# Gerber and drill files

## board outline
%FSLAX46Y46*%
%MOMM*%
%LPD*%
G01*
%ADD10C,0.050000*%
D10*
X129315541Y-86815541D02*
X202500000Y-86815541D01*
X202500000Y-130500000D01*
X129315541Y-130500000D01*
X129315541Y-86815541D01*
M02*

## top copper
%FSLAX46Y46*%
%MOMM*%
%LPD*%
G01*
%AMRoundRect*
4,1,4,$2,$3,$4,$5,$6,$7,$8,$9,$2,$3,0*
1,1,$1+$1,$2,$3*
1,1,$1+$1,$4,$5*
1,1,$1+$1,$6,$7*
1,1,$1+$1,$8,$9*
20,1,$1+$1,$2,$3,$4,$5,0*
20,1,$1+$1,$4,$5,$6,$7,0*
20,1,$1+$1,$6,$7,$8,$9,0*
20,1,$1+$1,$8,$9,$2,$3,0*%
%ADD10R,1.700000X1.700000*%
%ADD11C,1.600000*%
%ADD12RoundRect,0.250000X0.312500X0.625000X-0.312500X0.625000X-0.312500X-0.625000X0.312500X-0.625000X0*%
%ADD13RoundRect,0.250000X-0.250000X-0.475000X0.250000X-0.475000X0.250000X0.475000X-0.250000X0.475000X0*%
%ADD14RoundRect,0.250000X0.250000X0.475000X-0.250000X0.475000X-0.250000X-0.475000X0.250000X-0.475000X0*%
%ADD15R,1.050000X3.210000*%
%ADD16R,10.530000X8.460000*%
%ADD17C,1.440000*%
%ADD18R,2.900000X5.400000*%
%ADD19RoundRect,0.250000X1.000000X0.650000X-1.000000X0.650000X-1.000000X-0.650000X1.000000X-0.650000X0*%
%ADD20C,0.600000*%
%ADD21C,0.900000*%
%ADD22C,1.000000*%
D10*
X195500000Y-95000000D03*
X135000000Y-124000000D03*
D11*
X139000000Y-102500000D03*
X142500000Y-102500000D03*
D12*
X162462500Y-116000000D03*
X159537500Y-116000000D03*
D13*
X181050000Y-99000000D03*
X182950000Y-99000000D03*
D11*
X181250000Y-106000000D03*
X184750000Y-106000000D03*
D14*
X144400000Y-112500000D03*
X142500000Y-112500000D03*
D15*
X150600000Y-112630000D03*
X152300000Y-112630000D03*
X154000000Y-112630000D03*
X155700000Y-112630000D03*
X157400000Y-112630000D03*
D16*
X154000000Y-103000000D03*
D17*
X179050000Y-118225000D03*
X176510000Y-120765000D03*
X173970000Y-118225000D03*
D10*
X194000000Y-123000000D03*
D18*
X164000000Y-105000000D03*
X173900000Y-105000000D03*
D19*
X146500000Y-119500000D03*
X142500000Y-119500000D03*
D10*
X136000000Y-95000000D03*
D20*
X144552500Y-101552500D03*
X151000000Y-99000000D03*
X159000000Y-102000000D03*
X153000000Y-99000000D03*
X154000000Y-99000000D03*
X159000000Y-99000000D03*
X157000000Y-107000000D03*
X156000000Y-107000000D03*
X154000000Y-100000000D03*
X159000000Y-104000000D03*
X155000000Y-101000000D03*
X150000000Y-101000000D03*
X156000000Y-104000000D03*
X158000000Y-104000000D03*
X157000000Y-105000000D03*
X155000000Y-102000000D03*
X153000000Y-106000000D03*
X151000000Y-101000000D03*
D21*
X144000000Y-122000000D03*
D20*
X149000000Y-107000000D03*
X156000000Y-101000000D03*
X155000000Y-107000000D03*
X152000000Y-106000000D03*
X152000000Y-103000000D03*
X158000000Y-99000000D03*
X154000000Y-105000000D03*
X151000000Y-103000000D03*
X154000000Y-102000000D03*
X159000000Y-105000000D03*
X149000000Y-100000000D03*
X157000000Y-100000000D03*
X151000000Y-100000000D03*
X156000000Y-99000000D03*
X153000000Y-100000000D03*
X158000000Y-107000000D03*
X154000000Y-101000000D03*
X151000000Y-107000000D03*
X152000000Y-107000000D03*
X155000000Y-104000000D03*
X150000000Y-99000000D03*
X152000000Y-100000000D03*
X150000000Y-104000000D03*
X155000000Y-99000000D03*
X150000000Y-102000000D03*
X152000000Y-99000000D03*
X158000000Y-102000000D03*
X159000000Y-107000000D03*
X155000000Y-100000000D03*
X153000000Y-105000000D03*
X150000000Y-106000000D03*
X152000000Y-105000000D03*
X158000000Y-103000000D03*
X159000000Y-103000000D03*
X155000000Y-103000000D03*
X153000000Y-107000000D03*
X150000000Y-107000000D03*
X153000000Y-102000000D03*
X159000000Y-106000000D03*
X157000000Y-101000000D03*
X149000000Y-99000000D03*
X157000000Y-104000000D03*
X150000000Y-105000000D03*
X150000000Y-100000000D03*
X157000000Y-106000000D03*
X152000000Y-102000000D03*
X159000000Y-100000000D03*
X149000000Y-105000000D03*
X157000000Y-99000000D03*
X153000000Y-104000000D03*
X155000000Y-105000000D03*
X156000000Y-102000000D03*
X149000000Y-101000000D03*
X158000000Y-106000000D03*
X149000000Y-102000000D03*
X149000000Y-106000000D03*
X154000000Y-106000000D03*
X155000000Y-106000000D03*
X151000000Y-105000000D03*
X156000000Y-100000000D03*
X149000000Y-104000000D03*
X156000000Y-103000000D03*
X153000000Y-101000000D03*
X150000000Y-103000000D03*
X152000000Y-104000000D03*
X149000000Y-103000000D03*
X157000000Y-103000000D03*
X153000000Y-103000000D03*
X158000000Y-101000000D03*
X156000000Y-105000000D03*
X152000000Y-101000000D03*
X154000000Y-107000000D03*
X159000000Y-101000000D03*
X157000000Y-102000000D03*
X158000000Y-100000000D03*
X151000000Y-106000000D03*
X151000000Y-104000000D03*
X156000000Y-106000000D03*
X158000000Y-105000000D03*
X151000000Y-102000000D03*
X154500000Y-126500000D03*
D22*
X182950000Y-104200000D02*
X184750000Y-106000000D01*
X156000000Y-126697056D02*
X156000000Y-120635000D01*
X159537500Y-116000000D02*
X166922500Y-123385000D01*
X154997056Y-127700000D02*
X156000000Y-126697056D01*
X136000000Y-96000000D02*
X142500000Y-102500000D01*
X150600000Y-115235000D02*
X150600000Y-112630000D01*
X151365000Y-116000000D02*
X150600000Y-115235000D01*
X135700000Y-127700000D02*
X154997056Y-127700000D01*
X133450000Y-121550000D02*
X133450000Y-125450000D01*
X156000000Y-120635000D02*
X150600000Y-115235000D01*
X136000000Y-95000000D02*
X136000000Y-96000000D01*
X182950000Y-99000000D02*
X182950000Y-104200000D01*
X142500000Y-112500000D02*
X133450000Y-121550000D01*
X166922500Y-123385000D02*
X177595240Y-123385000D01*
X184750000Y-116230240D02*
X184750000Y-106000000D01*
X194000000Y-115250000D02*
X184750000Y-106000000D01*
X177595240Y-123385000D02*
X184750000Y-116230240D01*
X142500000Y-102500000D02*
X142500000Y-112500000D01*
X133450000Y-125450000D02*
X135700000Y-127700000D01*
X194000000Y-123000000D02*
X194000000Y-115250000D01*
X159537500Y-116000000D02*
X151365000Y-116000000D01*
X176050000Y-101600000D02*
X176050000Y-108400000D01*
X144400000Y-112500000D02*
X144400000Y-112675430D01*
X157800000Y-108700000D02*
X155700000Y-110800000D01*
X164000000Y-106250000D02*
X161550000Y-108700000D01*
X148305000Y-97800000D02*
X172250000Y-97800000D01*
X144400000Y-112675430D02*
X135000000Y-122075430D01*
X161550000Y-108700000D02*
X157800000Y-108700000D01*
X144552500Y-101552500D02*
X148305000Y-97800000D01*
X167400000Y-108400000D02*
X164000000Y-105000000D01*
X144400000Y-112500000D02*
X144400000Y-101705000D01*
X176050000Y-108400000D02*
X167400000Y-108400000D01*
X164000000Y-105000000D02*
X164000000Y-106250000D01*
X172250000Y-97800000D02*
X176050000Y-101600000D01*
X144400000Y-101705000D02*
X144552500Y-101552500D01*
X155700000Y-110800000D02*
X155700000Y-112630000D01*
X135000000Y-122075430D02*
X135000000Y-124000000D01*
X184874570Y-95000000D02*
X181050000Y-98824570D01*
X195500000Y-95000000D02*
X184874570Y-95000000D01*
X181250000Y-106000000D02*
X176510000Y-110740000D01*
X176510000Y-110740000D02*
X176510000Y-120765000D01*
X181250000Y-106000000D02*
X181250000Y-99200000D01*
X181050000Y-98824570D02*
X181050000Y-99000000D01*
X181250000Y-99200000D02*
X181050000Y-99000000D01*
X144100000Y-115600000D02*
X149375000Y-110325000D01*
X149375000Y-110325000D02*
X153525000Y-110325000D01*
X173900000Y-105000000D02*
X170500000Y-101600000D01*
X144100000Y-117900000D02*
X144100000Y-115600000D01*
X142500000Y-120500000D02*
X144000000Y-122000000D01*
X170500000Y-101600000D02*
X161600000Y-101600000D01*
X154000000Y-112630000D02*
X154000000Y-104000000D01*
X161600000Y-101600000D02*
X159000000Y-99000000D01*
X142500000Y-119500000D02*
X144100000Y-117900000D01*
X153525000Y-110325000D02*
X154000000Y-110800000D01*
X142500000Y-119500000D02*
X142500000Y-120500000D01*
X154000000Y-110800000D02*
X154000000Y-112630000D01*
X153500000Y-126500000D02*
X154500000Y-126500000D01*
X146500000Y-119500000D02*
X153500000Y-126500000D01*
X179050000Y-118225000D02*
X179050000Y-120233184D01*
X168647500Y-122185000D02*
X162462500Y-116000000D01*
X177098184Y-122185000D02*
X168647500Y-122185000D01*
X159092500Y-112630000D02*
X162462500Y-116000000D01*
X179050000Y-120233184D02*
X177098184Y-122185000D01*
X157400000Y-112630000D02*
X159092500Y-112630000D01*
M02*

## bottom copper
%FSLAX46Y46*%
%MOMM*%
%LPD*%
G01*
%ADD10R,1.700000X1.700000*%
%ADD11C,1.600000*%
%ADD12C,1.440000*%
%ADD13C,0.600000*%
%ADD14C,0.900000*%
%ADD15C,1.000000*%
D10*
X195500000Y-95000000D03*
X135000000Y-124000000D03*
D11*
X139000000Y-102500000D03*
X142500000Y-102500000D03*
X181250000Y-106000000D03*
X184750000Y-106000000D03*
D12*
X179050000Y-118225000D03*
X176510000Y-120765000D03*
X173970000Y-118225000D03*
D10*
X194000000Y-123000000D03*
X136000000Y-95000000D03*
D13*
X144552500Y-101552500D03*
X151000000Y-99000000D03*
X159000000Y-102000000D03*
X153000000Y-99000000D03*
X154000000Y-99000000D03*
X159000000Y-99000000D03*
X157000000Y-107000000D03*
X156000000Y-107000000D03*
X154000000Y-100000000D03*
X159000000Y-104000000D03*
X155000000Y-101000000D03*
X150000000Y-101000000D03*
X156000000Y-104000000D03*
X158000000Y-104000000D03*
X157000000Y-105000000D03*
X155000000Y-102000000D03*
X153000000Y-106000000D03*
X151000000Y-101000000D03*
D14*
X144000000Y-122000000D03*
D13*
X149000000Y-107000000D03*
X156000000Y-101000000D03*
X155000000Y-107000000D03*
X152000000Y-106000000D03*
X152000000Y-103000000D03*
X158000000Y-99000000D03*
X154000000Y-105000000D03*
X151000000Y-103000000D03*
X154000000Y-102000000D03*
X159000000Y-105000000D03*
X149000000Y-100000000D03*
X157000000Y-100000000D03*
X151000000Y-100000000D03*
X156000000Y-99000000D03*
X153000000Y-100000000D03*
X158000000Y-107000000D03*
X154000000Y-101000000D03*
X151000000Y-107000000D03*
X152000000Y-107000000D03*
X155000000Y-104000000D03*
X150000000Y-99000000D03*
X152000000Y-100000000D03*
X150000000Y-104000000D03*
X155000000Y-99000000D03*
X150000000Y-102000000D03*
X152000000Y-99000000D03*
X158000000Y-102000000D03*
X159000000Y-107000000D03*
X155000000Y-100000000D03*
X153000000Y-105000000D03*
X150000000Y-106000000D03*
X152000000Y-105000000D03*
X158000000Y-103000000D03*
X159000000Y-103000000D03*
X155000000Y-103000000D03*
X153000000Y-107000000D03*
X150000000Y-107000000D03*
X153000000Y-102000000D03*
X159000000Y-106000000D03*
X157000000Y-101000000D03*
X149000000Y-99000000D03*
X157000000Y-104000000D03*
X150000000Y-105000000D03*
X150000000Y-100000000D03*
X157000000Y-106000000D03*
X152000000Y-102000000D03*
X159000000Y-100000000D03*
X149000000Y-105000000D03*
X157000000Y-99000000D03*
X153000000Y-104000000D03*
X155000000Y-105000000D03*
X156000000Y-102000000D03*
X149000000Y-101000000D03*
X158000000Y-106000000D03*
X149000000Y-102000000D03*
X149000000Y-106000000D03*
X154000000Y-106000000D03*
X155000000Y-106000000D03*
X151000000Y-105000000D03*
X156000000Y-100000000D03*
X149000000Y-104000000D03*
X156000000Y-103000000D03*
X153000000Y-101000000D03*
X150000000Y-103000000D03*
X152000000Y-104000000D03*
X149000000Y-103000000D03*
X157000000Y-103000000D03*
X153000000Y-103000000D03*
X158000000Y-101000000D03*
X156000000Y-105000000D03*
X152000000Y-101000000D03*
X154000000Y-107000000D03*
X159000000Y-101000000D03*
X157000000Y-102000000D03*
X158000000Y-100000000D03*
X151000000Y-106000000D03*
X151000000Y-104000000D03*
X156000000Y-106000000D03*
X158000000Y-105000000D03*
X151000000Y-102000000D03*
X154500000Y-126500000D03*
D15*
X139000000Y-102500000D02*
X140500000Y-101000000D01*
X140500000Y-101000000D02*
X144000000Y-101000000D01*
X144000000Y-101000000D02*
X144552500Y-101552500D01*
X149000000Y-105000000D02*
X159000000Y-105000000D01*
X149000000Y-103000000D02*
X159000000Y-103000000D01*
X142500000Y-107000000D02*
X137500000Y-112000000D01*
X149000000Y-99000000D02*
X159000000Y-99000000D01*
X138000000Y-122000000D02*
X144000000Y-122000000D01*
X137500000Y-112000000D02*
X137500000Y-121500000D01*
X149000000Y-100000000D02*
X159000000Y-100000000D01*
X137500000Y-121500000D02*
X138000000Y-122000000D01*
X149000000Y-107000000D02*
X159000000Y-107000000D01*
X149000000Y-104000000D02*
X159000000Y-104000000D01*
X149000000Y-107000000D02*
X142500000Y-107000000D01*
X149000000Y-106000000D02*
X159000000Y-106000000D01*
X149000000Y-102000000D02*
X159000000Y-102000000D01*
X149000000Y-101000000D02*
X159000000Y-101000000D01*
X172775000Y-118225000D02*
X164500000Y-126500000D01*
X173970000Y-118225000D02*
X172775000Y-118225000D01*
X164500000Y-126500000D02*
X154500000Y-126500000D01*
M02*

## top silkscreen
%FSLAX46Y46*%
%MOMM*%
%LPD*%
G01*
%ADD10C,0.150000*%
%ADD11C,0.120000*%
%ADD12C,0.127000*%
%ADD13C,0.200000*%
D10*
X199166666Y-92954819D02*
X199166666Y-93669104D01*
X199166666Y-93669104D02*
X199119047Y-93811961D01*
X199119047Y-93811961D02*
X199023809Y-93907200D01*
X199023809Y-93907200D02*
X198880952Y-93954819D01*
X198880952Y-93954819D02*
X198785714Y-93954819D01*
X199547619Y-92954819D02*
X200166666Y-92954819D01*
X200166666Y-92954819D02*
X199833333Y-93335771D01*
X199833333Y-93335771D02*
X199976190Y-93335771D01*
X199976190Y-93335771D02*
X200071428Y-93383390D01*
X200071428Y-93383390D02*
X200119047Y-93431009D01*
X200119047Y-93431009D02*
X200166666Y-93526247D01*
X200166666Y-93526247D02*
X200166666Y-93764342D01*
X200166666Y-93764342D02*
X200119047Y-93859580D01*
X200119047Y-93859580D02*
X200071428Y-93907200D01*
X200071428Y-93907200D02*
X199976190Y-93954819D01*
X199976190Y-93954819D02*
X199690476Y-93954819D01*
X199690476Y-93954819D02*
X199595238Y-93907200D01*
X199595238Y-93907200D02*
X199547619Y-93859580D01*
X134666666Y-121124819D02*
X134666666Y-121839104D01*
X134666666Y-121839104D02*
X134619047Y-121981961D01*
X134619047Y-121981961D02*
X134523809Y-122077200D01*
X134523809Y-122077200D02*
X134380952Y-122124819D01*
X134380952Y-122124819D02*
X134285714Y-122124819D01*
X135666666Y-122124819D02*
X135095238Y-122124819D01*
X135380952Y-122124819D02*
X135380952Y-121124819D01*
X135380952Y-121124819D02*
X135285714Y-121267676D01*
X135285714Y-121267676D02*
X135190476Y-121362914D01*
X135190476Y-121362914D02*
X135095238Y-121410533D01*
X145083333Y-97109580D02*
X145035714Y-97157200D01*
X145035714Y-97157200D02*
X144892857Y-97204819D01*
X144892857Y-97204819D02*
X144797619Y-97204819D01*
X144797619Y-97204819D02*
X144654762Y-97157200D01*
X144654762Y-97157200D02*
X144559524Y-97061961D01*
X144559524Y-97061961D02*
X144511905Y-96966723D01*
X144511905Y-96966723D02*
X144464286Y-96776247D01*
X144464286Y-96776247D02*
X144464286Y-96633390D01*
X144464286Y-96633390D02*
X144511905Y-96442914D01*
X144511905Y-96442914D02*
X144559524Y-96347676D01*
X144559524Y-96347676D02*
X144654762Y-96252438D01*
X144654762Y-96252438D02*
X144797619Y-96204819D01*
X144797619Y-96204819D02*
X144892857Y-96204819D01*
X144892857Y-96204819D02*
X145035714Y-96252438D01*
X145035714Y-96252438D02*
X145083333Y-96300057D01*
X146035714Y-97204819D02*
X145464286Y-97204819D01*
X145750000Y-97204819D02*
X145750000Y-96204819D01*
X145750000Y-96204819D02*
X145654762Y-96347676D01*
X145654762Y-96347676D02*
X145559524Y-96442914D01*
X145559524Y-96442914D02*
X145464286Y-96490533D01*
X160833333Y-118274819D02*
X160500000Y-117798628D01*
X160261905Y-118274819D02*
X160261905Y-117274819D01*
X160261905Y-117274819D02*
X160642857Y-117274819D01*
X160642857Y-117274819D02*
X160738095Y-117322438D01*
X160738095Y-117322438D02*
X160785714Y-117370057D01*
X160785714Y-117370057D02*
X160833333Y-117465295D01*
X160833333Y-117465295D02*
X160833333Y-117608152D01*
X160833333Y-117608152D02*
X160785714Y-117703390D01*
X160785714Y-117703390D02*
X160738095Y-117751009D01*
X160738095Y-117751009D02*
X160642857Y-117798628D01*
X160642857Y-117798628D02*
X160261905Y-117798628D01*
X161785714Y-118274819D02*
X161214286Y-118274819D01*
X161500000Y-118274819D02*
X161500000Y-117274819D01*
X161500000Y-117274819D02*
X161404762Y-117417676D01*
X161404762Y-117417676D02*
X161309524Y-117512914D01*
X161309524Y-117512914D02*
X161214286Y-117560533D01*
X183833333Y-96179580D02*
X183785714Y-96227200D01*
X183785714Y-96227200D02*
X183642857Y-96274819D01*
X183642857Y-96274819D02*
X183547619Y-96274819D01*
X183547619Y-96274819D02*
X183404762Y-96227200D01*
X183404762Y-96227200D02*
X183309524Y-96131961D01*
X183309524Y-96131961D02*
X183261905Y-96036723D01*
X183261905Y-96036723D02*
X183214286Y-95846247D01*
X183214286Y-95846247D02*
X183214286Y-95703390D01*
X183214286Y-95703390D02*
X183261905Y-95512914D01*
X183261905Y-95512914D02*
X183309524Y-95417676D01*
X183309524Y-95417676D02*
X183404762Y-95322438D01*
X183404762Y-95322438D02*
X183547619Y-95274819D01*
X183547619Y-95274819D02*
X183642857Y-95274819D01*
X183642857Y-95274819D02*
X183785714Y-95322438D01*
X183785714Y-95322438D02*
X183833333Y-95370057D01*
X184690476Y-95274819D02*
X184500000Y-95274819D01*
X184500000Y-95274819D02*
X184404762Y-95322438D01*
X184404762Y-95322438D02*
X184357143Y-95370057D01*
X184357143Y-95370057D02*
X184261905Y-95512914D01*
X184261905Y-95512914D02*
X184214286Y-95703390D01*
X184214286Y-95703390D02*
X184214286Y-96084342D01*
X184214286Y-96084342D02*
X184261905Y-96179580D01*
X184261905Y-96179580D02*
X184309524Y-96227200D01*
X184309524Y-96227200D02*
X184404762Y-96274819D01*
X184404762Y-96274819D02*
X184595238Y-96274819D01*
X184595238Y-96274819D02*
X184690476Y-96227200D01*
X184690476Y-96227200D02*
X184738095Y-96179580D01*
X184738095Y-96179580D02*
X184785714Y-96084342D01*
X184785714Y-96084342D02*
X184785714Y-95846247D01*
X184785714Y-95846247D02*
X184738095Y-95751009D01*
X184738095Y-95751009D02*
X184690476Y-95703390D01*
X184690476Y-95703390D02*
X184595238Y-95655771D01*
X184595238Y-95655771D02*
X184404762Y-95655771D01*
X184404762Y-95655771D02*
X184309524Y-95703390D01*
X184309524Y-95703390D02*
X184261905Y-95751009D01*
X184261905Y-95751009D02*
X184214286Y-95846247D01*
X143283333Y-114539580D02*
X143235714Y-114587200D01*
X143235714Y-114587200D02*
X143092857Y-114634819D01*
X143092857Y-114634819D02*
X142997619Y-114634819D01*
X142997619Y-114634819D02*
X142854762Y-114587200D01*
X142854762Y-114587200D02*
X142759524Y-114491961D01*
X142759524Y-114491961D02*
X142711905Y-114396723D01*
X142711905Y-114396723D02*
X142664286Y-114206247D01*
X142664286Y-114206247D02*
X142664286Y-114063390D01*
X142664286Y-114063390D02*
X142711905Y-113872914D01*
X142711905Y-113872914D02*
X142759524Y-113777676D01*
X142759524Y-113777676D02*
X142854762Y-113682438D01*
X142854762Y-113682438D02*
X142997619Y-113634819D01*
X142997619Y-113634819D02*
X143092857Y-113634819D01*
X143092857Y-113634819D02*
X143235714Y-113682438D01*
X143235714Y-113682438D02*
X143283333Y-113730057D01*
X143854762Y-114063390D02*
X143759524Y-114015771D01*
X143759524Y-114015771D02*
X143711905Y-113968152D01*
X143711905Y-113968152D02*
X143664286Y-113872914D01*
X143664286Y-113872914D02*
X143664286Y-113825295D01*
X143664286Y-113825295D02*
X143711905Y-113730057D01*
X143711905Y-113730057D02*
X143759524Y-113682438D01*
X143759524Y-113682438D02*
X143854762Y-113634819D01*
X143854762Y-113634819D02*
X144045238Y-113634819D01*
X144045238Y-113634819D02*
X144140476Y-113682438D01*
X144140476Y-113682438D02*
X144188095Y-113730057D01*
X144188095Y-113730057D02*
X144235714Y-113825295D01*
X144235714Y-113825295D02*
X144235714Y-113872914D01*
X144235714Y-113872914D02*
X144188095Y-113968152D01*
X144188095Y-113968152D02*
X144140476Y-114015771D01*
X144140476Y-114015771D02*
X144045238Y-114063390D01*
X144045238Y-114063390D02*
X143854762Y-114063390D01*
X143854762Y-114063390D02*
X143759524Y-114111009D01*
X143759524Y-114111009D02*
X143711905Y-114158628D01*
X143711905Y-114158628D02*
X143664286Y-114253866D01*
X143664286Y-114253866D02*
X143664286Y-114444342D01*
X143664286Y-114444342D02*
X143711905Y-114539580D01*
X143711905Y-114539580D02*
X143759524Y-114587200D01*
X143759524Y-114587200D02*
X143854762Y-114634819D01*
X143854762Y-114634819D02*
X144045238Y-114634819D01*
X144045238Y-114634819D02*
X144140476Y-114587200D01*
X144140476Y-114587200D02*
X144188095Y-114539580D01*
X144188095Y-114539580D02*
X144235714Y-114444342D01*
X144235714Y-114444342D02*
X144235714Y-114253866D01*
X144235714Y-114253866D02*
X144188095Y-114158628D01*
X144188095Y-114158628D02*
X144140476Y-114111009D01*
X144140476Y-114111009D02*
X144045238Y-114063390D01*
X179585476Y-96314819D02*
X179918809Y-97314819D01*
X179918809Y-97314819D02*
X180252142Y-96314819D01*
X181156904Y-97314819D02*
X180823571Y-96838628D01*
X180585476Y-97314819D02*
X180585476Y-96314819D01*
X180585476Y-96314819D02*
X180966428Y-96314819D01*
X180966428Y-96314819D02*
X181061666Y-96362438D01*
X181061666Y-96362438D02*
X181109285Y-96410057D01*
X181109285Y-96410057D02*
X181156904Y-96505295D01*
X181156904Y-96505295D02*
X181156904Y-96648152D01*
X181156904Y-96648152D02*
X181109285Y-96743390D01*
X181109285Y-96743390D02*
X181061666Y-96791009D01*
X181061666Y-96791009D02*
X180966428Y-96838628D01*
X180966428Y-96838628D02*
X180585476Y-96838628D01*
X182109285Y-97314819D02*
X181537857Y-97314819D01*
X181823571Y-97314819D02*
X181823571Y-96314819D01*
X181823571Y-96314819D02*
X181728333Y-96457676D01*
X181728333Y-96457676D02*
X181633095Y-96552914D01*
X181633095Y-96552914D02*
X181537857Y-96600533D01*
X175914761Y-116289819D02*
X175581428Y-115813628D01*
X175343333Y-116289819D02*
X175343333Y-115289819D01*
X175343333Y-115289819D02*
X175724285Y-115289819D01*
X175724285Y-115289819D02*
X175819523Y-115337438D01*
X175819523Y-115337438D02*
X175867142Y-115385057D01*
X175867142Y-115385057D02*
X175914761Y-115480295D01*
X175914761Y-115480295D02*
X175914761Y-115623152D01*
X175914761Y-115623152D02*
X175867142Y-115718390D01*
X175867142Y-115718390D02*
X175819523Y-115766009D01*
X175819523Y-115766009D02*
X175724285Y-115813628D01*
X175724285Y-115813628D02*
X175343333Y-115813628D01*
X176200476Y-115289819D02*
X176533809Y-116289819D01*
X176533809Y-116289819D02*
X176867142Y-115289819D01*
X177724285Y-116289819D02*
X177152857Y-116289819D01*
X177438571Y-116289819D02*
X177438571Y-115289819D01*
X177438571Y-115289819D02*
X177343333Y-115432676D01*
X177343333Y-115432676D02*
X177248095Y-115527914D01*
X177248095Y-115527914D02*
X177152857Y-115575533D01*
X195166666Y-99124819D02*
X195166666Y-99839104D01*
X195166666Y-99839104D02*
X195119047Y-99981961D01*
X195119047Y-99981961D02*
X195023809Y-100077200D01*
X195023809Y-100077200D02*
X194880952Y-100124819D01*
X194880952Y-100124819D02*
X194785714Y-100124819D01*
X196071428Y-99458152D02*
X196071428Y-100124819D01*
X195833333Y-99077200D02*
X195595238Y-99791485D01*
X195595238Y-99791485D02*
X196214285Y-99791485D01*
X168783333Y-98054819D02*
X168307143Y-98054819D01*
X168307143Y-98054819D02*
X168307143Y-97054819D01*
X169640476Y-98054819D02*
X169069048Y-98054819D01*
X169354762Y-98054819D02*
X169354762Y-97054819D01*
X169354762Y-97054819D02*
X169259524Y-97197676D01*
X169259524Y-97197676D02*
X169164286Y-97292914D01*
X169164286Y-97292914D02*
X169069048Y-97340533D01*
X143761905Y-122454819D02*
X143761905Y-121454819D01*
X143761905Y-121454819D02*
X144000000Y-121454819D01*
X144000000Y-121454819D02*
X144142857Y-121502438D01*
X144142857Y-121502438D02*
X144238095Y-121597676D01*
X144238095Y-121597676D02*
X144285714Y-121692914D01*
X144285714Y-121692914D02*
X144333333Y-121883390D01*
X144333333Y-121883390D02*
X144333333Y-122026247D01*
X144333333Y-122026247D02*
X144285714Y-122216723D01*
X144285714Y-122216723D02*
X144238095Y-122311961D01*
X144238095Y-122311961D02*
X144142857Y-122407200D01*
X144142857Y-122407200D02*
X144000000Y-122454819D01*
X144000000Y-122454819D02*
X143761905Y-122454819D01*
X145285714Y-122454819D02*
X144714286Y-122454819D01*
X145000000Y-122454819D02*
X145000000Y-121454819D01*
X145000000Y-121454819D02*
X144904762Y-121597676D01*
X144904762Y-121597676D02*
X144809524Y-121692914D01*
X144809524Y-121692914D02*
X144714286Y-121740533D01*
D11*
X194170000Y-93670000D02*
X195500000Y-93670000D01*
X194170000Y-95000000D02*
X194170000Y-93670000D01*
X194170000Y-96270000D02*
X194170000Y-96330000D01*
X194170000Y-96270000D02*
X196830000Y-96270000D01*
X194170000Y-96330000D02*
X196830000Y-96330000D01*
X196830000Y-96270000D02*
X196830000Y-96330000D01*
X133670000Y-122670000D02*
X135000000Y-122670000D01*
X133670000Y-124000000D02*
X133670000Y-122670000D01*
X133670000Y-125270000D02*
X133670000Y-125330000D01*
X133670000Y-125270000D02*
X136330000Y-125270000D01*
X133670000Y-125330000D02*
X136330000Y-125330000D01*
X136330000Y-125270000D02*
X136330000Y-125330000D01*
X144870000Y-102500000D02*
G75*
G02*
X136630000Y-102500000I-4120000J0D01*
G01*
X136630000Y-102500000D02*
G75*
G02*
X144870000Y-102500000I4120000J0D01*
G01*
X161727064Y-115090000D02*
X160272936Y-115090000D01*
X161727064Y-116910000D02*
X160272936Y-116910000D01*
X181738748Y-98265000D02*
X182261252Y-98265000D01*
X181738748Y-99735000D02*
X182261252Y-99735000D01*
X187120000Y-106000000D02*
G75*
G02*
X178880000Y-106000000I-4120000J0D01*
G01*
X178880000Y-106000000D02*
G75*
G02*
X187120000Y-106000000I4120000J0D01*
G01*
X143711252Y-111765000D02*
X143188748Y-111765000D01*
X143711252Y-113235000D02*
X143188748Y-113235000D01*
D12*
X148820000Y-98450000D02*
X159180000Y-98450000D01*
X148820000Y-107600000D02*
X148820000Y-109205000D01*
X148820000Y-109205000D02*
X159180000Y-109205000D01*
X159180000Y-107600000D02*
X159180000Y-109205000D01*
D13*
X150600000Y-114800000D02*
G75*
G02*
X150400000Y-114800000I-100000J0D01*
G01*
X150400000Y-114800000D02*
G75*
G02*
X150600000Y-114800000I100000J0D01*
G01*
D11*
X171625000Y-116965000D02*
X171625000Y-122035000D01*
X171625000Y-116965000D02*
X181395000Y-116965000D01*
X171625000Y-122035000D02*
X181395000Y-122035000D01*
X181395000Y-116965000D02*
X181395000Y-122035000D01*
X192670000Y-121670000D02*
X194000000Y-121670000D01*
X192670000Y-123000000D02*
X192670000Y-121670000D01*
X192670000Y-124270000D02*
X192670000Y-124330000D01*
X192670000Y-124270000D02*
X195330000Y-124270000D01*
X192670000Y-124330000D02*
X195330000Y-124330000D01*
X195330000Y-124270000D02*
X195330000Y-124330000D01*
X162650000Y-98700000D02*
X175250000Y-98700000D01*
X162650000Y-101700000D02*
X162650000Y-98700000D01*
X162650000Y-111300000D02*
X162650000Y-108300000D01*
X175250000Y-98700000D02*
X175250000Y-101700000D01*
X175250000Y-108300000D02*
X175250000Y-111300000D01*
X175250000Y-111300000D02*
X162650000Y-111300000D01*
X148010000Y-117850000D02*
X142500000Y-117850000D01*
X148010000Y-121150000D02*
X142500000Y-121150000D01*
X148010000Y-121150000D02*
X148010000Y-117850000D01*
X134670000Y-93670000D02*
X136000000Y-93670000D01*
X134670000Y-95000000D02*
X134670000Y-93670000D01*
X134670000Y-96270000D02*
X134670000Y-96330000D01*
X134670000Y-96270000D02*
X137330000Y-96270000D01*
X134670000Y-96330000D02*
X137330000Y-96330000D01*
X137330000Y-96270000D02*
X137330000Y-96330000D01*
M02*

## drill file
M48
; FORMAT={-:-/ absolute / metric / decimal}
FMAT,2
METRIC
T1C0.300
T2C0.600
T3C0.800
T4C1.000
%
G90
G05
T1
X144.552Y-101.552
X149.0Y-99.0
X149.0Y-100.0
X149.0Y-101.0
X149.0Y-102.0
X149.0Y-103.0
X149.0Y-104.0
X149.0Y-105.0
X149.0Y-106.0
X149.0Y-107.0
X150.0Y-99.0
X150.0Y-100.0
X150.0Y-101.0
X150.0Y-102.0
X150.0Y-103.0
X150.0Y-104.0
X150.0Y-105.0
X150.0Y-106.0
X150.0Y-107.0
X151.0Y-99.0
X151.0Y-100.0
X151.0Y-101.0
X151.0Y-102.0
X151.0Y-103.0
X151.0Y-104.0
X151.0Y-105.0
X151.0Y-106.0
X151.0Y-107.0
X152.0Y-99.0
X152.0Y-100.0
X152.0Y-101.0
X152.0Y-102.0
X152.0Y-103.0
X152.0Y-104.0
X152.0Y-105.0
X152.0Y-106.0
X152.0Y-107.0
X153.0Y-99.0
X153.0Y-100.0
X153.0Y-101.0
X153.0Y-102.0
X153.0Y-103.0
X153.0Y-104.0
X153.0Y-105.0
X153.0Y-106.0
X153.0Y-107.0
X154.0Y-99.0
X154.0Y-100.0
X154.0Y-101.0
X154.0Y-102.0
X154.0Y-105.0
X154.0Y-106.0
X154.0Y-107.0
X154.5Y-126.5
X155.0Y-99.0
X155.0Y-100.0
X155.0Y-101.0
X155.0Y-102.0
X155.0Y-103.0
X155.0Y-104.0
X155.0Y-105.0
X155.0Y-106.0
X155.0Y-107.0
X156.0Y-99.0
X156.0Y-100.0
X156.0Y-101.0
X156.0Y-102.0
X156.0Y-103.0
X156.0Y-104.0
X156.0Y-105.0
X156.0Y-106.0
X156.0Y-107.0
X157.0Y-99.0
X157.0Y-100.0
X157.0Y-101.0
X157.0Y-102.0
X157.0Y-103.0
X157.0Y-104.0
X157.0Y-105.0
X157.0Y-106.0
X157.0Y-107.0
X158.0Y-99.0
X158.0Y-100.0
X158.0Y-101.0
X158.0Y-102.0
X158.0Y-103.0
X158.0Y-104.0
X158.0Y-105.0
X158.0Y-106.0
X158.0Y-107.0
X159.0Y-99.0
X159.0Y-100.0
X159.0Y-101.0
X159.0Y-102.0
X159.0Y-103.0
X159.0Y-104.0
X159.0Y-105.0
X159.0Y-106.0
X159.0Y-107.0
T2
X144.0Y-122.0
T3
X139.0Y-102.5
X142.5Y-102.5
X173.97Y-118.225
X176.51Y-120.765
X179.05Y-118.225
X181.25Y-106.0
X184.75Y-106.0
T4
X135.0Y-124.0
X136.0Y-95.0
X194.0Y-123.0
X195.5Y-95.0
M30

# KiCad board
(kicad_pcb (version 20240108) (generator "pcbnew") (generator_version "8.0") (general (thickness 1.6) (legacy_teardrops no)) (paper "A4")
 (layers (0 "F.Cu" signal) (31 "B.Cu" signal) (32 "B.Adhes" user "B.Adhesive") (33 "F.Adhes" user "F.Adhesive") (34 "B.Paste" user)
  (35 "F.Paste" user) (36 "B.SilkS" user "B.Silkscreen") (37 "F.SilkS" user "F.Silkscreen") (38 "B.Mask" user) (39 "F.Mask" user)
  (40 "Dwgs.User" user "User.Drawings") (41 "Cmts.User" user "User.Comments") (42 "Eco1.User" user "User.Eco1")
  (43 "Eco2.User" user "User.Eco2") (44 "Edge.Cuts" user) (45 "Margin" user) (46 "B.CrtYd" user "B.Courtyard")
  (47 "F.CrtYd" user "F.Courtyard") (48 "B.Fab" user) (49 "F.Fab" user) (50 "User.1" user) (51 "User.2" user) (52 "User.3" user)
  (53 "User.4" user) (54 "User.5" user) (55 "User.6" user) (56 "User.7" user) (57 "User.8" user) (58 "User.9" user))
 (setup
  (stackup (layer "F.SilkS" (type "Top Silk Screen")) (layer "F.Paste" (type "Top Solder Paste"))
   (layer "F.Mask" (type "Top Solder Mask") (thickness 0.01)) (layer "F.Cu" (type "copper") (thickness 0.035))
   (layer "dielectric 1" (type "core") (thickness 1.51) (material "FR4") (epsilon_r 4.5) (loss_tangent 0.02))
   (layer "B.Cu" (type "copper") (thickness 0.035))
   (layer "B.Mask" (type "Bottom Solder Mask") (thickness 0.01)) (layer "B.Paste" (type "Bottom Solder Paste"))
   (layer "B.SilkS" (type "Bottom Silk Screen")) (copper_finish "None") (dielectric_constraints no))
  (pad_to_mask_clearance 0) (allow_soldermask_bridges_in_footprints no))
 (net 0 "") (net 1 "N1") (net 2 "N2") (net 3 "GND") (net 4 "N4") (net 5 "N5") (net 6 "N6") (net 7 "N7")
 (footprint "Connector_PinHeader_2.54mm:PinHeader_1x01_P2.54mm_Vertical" (layer "F.Cu") (at 195.5 95)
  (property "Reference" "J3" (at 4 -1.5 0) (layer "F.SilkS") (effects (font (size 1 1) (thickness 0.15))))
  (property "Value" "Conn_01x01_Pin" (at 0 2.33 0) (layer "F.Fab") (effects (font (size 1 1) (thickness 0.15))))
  (fp_line (start -1.33 -1.33) (end 0 -1.33) (stroke (width 0.12) (type solid)) (layer "F.SilkS"))
  (fp_line (start -1.33 0) (end -1.33 -1.33) (stroke (width 0.12) (type solid)) (layer "F.SilkS"))
  (fp_line (start -1.33 1.27) (end -1.33 1.33) (stroke (width 0.12) (type solid)) (layer "F.SilkS"))
  (fp_line (start -1.33 1.27) (end 1.33 1.27) (stroke (width 0.12) (type solid)) (layer "F.SilkS"))
  (fp_line (start -1.33 1.33) (end 1.33 1.33) (stroke (width 0.12) (type solid)) (layer "F.SilkS"))
  (fp_line (start 1.33 1.27) (end 1.33 1.33) (stroke (width 0.12) (type solid)) (layer "F.SilkS"))
  (pad "1" thru_hole rect (at 0 0) (size 1.7 1.7) (drill 1) (layers "*.Cu" "*.Mask") (remove_unused_layers no) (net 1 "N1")))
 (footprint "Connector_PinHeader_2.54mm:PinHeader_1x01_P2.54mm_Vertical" (layer "F.Cu") (at 135 124)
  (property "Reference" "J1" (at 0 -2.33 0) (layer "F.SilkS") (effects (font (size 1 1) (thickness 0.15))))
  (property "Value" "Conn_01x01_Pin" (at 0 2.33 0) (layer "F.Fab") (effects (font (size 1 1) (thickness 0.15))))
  (fp_line (start -1.33 -1.33) (end 0 -1.33) (stroke (width 0.12) (type solid)) (layer "F.SilkS"))
  (fp_line (start -1.33 0) (end -1.33 -1.33) (stroke (width 0.12) (type solid)) (layer "F.SilkS"))
  (fp_line (start -1.33 1.27) (end -1.33 1.33) (stroke (width 0.12) (type solid)) (layer "F.SilkS"))
  (fp_line (start -1.33 1.27) (end 1.33 1.27) (stroke (width 0.12) (type solid)) (layer "F.SilkS"))
  (fp_line (start -1.33 1.33) (end 1.33 1.33) (stroke (width 0.12) (type solid)) (layer "F.SilkS"))
  (fp_line (start 1.33 1.27) (end 1.33 1.33) (stroke (width 0.12) (type solid)) (layer "F.SilkS"))
  (pad "1" thru_hole rect (at 0 0) (size 1.7 1.7) (drill 1) (layers "*.Cu" "*.Mask") (remove_unused_layers no) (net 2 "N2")))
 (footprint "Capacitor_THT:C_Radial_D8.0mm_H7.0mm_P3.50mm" (layer "F.Cu") (at 139 102.5)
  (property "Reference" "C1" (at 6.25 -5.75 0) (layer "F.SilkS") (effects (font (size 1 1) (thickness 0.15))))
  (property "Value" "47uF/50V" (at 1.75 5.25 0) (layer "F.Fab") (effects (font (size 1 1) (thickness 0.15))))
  (fp_circle (center 1.75 0) (end 5.87 0) (stroke (width 0.12) (type solid)) (fill none) (layer "F.SilkS"))
  (pad "1" thru_hole circle (at 0 0) (size 1.6 1.6) (drill 0.8) (layers "*.Cu" "*.Mask") (remove_unused_layers no) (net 2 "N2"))
  (pad "2" thru_hole circle (at 3.5 0) (size 1.6 1.6) (drill 0.8) (layers "*.Cu" "*.Mask") (remove_unused_layers no) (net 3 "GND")))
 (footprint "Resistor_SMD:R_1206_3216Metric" (layer "F.Cu") (at 161 116 180)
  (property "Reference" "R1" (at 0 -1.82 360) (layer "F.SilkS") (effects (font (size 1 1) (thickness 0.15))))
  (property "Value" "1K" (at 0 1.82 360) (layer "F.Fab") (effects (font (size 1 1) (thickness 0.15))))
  (fp_line (start -0.727064 0.91) (end 0.727064 0.91) (stroke (width 0.12) (type solid)) (layer "F.SilkS"))
  (fp_line (start -0.727064 -0.91) (end 0.727064 -0.91) (stroke (width 0.12) (type solid)) (layer "F.SilkS"))
  (pad "1" smd roundrect (at -1.4625 0 180) (size 1.125 1.75) (layers "F.Cu" "F.Paste" "F.Mask") (roundrect_rratio 0.222222) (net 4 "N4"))
  (pad "2" smd roundrect (at 1.4625 0 180) (size 1.125 1.75) (layers "F.Cu" "F.Paste" "F.Mask") (roundrect_rratio 0.222222) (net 3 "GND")))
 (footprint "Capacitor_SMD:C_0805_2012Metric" (layer "F.Cu") (at 182 99)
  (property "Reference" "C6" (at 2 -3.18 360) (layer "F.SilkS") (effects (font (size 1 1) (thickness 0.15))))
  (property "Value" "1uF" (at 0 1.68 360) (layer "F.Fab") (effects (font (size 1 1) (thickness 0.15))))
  (fp_line (start -0.261252 -0.735) (end 0.261252 -0.735) (stroke (width 0.12) (type solid)) (layer "F.SilkS"))
  (fp_line (start -0.261252 0.735) (end 0.261252 0.735) (stroke (width 0.12) (type solid)) (layer "F.SilkS"))
  (pad "1" smd roundrect (at -0.95 0) (size 1 1.45) (layers "F.Cu" "F.Paste" "F.Mask") (roundrect_rratio 0.25) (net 1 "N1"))
  (pad "2" smd roundrect (at 0.95 0) (size 1 1.45) (layers "F.Cu" "F.Paste" "F.Mask") (roundrect_rratio 0.25) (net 3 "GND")))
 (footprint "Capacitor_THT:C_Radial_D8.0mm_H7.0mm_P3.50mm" (layer "F.Cu") (at 181.25 106)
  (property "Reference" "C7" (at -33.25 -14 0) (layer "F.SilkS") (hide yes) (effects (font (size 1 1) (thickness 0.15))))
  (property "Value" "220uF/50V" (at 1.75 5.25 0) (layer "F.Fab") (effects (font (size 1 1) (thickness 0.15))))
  (fp_circle (center 1.75 0) (end 5.87 0) (stroke (width 0.12) (type solid)) (fill none) (layer "F.SilkS"))
  (pad "1" thru_hole circle (at 0 0) (size 1.6 1.6) (drill 0.8) (layers "*.Cu" "*.Mask") (remove_unused_layers no) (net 1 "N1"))
  (pad "2" thru_hole circle (at 3.5 0) (size 1.6 1.6) (drill 0.8) (layers "*.Cu" "*.Mask") (remove_unused_layers no) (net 3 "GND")))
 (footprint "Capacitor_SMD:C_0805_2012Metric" (layer "F.Cu") (at 143.45 112.5 180)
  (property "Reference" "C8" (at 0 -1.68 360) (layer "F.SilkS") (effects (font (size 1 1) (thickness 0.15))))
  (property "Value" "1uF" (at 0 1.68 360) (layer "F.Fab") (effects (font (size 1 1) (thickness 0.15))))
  (fp_line (start -0.261252 0.735) (end 0.261252 0.735) (stroke (width 0.12) (type solid)) (layer "F.SilkS"))
  (fp_line (start -0.261252 -0.735) (end 0.261252 -0.735) (stroke (width 0.12) (type solid)) (layer "F.SilkS"))
  (pad "1" smd roundrect (at -0.95 0 180) (size 1 1.45) (layers "F.Cu" "F.Paste" "F.Mask") (roundrect_rratio 0.25) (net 2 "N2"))
  (pad "2" smd roundrect (at 0.95 0 180) (size 1 1.45) (layers "F.Cu" "F.Paste" "F.Mask") (roundrect_rratio 0.25) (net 3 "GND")))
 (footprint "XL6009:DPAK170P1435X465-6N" (layer "F.Cu") (at 154 106.5 90)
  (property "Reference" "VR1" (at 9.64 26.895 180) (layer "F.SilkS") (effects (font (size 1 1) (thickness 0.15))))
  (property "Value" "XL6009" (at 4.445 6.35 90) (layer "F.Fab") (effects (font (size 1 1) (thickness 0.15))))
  (fp_line (start 8.05 -5.18) (end 8.05 5.18) (stroke (width 0.127) (type solid)) (layer "F.SilkS"))
  (fp_line (start -1.1 -5.18) (end -2.705 -5.18) (stroke (width 0.127) (type solid)) (layer "F.SilkS"))
  (fp_line (start -2.705 -5.18) (end -2.705 5.18) (stroke (width 0.127) (type solid)) (layer "F.SilkS"))
  (fp_line (start -1.1 5.18) (end -2.705 5.18) (stroke (width 0.127) (type solid)) (layer "F.SilkS"))
  (fp_circle (center -8.3 -3.5) (end -8.2 -3.5) (stroke (width 0.2) (type solid)) (fill none) (layer "F.SilkS"))
  (pad "1" smd rect (at -6.13 -3.4 90) (size 3.21 1.05) (layers "F.Cu" "F.Paste" "F.Mask") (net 3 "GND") (solder_mask_margin 0.102))
  (pad "2" smd rect (at -6.13 -1.7 90) (size 3.21 1.05) (layers "F.Cu" "F.Paste" "F.Mask") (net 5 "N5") (solder_mask_margin 0.102))
  (pad "3" smd rect (at -6.13 0 90) (size 3.21 1.05) (layers "F.Cu" "F.Paste" "F.Mask") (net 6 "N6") (solder_mask_margin 0.102))
  (pad "4" smd rect (at -6.13 1.7 90) (size 3.21 1.05) (layers "F.Cu" "F.Paste" "F.Mask") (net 2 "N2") (solder_mask_margin 0.102))
  (pad "5" smd rect (at -6.13 3.4 90) (size 3.21 1.05) (layers "F.Cu" "F.Paste" "F.Mask") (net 4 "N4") (solder_mask_margin 0.102))
  (pad "6" smd rect (at 3.5 0 90) (size 8.46 10.53) (layers "F.Cu" "F.Mask") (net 6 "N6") (solder_mask_margin 0.102)))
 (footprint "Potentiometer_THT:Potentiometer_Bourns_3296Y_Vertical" (layer "F.Cu") (at 179.05 118.225)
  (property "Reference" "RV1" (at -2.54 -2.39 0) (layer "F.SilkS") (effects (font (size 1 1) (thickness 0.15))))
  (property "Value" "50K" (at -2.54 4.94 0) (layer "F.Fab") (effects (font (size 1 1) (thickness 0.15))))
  (fp_line (start -7.425 -1.26) (end -7.425 3.81) (stroke (width 0.12) (type solid)) (layer "F.SilkS"))
  (fp_line (start -7.425 -1.26) (end 2.345 -1.26) (stroke (width 0.12) (type solid)) (layer "F.SilkS"))
  (fp_line (start -7.425 3.81) (end 2.345 3.81) (stroke (width 0.12) (type solid)) (layer "F.SilkS"))
  (fp_line (start 2.345 -1.26) (end 2.345 3.81) (stroke (width 0.12) (type solid)) (layer "F.SilkS"))
  (pad "1" thru_hole circle (at 0 0) (size 1.44 1.44) (drill 0.8) (layers "*.Cu" "*.Mask") (remove_unused_layers no) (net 4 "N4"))
  (pad "2" thru_hole circle (at -2.54 2.54) (size 1.44 1.44) (drill 0.8) (layers "*.Cu" "*.Mask") (remove_unused_layers no) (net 1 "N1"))
  (pad "3" thru_hole circle (at -5.08 0) (size 1.44 1.44) (drill 0.8) (layers "*.Cu" "*.Mask") (remove_unused_layers no) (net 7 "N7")))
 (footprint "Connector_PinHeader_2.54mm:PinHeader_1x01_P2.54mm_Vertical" (layer "F.Cu") (at 194 123)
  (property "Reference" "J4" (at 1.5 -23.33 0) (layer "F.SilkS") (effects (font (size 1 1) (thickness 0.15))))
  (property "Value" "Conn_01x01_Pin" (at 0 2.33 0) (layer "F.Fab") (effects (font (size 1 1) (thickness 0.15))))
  (fp_line (start -1.33 -1.33) (end 0 -1.33) (stroke (width 0.12) (type solid)) (layer "F.SilkS"))
  (fp_line (start -1.33 0) (end -1.33 -1.33) (stroke (width 0.12) (type solid)) (layer "F.SilkS"))
  (fp_line (start -1.33 1.27) (end -1.33 1.33) (stroke (width 0.12) (type solid)) (layer "F.SilkS"))
  (fp_line (start -1.33 1.27) (end 1.33 1.27) (stroke (width 0.12) (type solid)) (layer "F.SilkS"))
  (fp_line (start -1.33 1.33) (end 1.33 1.33) (stroke (width 0.12) (type solid)) (layer "F.SilkS"))
  (fp_line (start 1.33 1.27) (end 1.33 1.33) (stroke (width 0.12) (type solid)) (layer "F.SilkS"))
  (pad "1" thru_hole rect (at 0 0) (size 1.7 1.7) (drill 1) (layers "*.Cu" "*.Mask") (remove_unused_layers no) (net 3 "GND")))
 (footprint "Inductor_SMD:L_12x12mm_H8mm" (layer "F.Cu") (at 168.95 105)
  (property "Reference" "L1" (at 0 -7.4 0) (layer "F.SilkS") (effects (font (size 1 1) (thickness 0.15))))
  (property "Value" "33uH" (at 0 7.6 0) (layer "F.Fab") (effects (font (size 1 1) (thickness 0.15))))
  (fp_line (start -6.3 -6.3) (end 6.3 -6.3) (stroke (width 0.12) (type solid)) (layer "F.SilkS"))
  (fp_line (start -6.3 -3.3) (end -6.3 -6.3) (stroke (width 0.12) (type solid)) (layer "F.SilkS"))
  (fp_line (start -6.3 6.3) (end -6.3 3.3) (stroke (width 0.12) (type solid)) (layer "F.SilkS"))
  (fp_line (start 6.3 -6.3) (end 6.3 -3.3) (stroke (width 0.12) (type solid)) (layer "F.SilkS"))
  (fp_line (start 6.3 3.3) (end 6.3 6.3) (stroke (width 0.12) (type solid)) (layer "F.SilkS"))
  (fp_line (start 6.3 6.3) (end -6.3 6.3) (stroke (width 0.12) (type solid)) (layer "F.SilkS"))
  (pad "1" smd rect (at -4.95 0) (size 2.9 5.4) (layers "F.Cu" "F.Paste" "F.Mask") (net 2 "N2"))
  (pad "2" smd rect (at 4.95 0) (size 2.9 5.4) (layers "F.Cu" "F.Paste" "F.Mask") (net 6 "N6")))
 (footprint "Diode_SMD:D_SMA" (layer "F.Cu") (at 144.5 119.5 180)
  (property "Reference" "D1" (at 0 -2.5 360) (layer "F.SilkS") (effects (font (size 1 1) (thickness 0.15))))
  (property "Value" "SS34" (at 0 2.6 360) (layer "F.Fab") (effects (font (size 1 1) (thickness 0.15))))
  (fp_line (start -3.51 1.65) (end 2 1.65) (stroke (width 0.12) (type solid)) (layer "F.SilkS"))
  (fp_line (start -3.51 -1.65) (end 2 -1.65) (stroke (width 0.12) (type solid)) (layer "F.SilkS"))
  (fp_line (start -3.51 -1.65) (end -3.51 1.65) (stroke (width 0.12) (type solid)) (layer "F.SilkS"))
  (pad "1" smd roundrect (at -2 0 180) (size 2.5 1.8) (layers "F.Cu" "F.Paste" "F.Mask") (roundrect_rratio 0.1388888889) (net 7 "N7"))
  (pad "2" smd roundrect (at 2 0 180) (size 2.5 1.8) (layers "F.Cu" "F.Paste" "F.Mask") (roundrect_rratio 0.1388888889) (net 6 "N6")))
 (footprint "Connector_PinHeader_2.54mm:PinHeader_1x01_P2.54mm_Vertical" (layer "F.Cu") (at 136 95)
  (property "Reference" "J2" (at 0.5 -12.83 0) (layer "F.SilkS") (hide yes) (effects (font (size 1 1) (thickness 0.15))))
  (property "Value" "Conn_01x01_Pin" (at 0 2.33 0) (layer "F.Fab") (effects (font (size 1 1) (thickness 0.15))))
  (fp_line (start -1.33 -1.33) (end 0 -1.33) (stroke (width 0.12) (type solid)) (layer "F.SilkS"))
  (fp_line (start -1.33 0) (end -1.33 -1.33) (stroke (width 0.12) (type solid)) (layer "F.SilkS"))
  (fp_line (start -1.33 1.27) (end -1.33 1.33) (stroke (width 0.12) (type solid)) (layer "F.SilkS"))
  (fp_line (start -1.33 1.27) (end 1.33 1.27) (stroke (width 0.12) (type solid)) (layer "F.SilkS"))
  (fp_line (start -1.33 1.33) (end 1.33 1.33) (stroke (width 0.12) (type solid)) (layer "F.SilkS"))
  (fp_line (start 1.33 1.27) (end 1.33 1.33) (stroke (width 0.12) (type solid)) (layer "F.SilkS"))
  (pad "1" thru_hole rect (at 0 0) (size 1.7 1.7) (drill 1) (layers "*.Cu" "*.Mask") (remove_unused_layers no) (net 3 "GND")))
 (gr_rect (start 129.315541 86.815541) (end 202.5 130.5) (stroke (width 0.05) (type default)) (fill none) (layer "Edge.Cuts"))
 (segment (start 182.95 104.2) (end 184.75 106) (width 1) (layer "F.Cu") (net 3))
 (segment (start 156 126.697056) (end 156 120.635) (width 1) (layer "F.Cu") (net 3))
 (segment (start 159.5375 116) (end 166.9225 123.385) (width 1) (layer "F.Cu") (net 3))
 (segment (start 154.997056 127.7) (end 156 126.697056) (width 1) (layer "F.Cu") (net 3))
 (segment (start 136 96) (end 142.5 102.5) (width 1) (layer "F.Cu") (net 3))
 (segment (start 150.6 115.235) (end 150.6 112.63) (width 1) (layer "F.Cu") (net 3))
 (segment (start 151.365 116) (end 150.6 115.235) (width 1) (layer "F.Cu") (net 3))
 (segment (start 135.7 127.7) (end 154.997056 127.7) (width 1) (layer "F.Cu") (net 3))
 (segment (start 133.45 121.55) (end 133.45 125.45) (width 1) (layer "F.Cu") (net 3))
 (segment (start 156 120.635) (end 150.6 115.235) (width 1) (layer "F.Cu") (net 3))
 (segment (start 136 95) (end 136 96) (width 1) (layer "F.Cu") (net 3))
 (segment (start 182.95 99) (end 182.95 104.2) (width 1) (layer "F.Cu") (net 3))
 (segment (start 142.5 112.5) (end 133.45 121.55) (width 1) (layer "F.Cu") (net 3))
 (segment (start 166.9225 123.385) (end 177.59524 123.385) (width 1) (layer "F.Cu") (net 3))
 (segment (start 184.75 116.23024) (end 184.75 106) (width 1) (layer "F.Cu") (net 3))
 (segment (start 194 115.25) (end 184.75 106) (width 1) (layer "F.Cu") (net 3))
 (segment (start 177.59524 123.385) (end 184.75 116.23024) (width 1) (layer "F.Cu") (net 3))
 (segment (start 142.5 102.5) (end 142.5 112.5) (width 1) (layer "F.Cu") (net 3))
 (segment (start 133.45 125.45) (end 135.7 127.7) (width 1) (layer "F.Cu") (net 3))
 (segment (start 194 123) (end 194 115.25) (width 1) (layer "F.Cu") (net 3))
 (segment (start 159.5375 116) (end 151.365 116) (width 1) (layer "F.Cu") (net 3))
 (segment (start 176.05 101.6) (end 176.05 108.4) (width 1) (layer "F.Cu") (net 2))
 (segment (start 144.4 112.5) (end 144.4 112.67543) (width 1) (layer "F.Cu") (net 2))
 (segment (start 157.8 108.7) (end 155.7 110.8) (width 1) (layer "F.Cu") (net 2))
 (segment (start 164 106.25) (end 161.55 108.7) (width 1) (layer "F.Cu") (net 2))
 (segment (start 148.305 97.8) (end 172.25 97.8) (width 1) (layer "F.Cu") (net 2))
 (segment (start 144.4 112.67543) (end 135 122.07543) (width 1) (layer "F.Cu") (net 2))
 (segment (start 161.55 108.7) (end 157.8 108.7) (width 1) (layer "F.Cu") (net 2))
 (segment (start 144.5525 101.5525) (end 148.305 97.8) (width 1) (layer "F.Cu") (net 2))
 (segment (start 167.4 108.4) (end 164 105) (width 1) (layer "F.Cu") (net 2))
 (segment (start 144.4 112.5) (end 144.4 101.705) (width 1) (layer "F.Cu") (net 2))
 (segment (start 176.05 108.4) (end 167.4 108.4) (width 1) (layer "F.Cu") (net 2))
 (segment (start 164 105) (end 164 106.25) (width 1) (layer "F.Cu") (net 2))
 (segment (start 172.25 97.8) (end 176.05 101.6) (width 1) (layer "F.Cu") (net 2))
 (segment (start 144.4 101.705) (end 144.5525 101.5525) (width 1) (layer "F.Cu") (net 2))
 (segment (start 155.7 110.8) (end 155.7 112.63) (width 1) (layer "F.Cu") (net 2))
 (segment (start 135 122.07543) (end 135 124) (width 1) (layer "F.Cu") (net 2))
 (via (at 144.5525 101.5525) (size 0.6) (drill 0.3) (layers "F.Cu" "B.Cu") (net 2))
 (segment (start 139 102.5) (end 140.5 101) (width 1) (layer "B.Cu") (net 2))
 (segment (start 140.5 101) (end 144 101) (width 1) (layer "B.Cu") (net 2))
 (segment (start 144 101) (end 144.5525 101.5525) (width 1) (layer "B.Cu") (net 2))
 (segment (start 184.87457 95) (end 181.05 98.82457) (width 1) (layer "F.Cu") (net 1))
 (segment (start 195.5 95) (end 184.87457 95) (width 1) (layer "F.Cu") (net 1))
 (segment (start 181.25 106) (end 176.51 110.74) (width 1) (layer "F.Cu") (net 1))
 (segment (start 176.51 110.74) (end 176.51 120.765) (width 1) (layer "F.Cu") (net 1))
 (segment (start 181.25 106) (end 181.25 99.2) (width 1) (layer "F.Cu") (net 1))
 (segment (start 181.05 98.82457) (end 181.05 99) (width 1) (layer "F.Cu") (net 1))
 (segment (start 181.25 99.2) (end 181.05 99) (width 1) (layer "F.Cu") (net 1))
 (segment (start 144.1 115.6) (end 149.375 110.325) (width 1) (layer "F.Cu") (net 6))
 (segment (start 149.375 110.325) (end 153.525 110.325) (width 1) (layer "F.Cu") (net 6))
 (segment (start 173.9 105) (end 170.5 101.6) (width 1) (layer "F.Cu") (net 6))
 (segment (start 144.1 117.9) (end 144.1 115.6) (width 1) (layer "F.Cu") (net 6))
 (segment (start 142.5 120.5) (end 144 122) (width 1) (layer "F.Cu") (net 6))
 (segment (start 170.5 101.6) (end 161.6 101.6) (width 1) (layer "F.Cu") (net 6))
 (segment (start 154 112.63) (end 154 104) (width 1) (layer "F.Cu") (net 6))
 (segment (start 161.6 101.6) (end 159 99) (width 1) (layer "F.Cu") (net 6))
 (segment (start 142.5 119.5) (end 144.1 117.9) (width 1) (layer "F.Cu") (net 6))
 (segment (start 153.525 110.325) (end 154 110.8) (width 1) (layer "F.Cu") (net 6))
 (segment (start 142.5 119.5) (end 142.5 120.5) (width 1) (layer "F.Cu") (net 6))
 (segment (start 154 110.8) (end 154 112.63) (width 1) (layer "F.Cu") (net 6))
 (via (at 151 99) (size 0.6) (drill 0.3) (layers "F.Cu" "B.Cu") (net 6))
 (via (at 159 102) (size 0.6) (drill 0.3) (layers "F.Cu" "B.Cu") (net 6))
 (via (at 153 99) (size 0.6) (drill 0.3) (layers "F.Cu" "B.Cu") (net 6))
 (via (at 154 99) (size 0.6) (drill 0.3) (layers "F.Cu" "B.Cu") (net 6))
 (via (at 159 99) (size 0.6) (drill 0.3) (layers "F.Cu" "B.Cu") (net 6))
 (via (at 157 107) (size 0.6) (drill 0.3) (layers "F.Cu" "B.Cu") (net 6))
 (via (at 156 107) (size 0.6) (drill 0.3) (layers "F.Cu" "B.Cu") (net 6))
 (via (at 154 100) (size 0.6) (drill 0.3) (layers "F.Cu" "B.Cu") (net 6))
 (via (at 159 104) (size 0.6) (drill 0.3) (layers "F.Cu" "B.Cu") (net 6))
 (via (at 155 101) (size 0.6) (drill 0.3) (layers "F.Cu" "B.Cu") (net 6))
 (via (at 150 101) (size 0.6) (drill 0.3) (layers "F.Cu" "B.Cu") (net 6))
 (via (at 156 104) (size 0.6) (drill 0.3) (layers "F.Cu" "B.Cu") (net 6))
 (via (at 158 104) (size 0.6) (drill 0.3) (layers "F.Cu" "B.Cu") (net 6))
 (via (at 157 105) (size 0.6) (drill 0.3) (layers "F.Cu" "B.Cu") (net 6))
 (via (at 155 102) (size 0.6) (drill 0.3) (layers "F.Cu" "B.Cu") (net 6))
 (via (at 153 106) (size 0.6) (drill 0.3) (layers "F.Cu" "B.Cu") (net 6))
 (via (at 151 101) (size 0.6) (drill 0.3) (layers "F.Cu" "B.Cu") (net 6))
 (via (at 144 122) (size 0.9) (drill 0.6) (layers "F.Cu" "B.Cu") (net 6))
 (via (at 149 107) (size 0.6) (drill 0.3) (layers "F.Cu" "B.Cu") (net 6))
 (via (at 156 101) (size 0.6) (drill 0.3) (layers "F.Cu" "B.Cu") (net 6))
 (via (at 155 107) (size 0.6) (drill 0.3) (layers "F.Cu" "B.Cu") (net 6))
 (via (at 152 106) (size 0.6) (drill 0.3) (layers "F.Cu" "B.Cu") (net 6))
 (via (at 152 103) (size 0.6) (drill 0.3) (layers "F.Cu" "B.Cu") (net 6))
 (via (at 158 99) (size 0.6) (drill 0.3) (layers "F.Cu" "B.Cu") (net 6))
 (via (at 154 105) (size 0.6) (drill 0.3) (layers "F.Cu" "B.Cu") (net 6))
 (via (at 151 103) (size 0.6) (drill 0.3) (layers "F.Cu" "B.Cu") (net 6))
 (via (at 154 102) (size 0.6) (drill 0.3) (layers "F.Cu" "B.Cu") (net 6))
 (via (at 159 105) (size 0.6) (drill 0.3) (layers "F.Cu" "B.Cu") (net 6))
 (via (at 149 100) (size 0.6) (drill 0.3) (layers "F.Cu" "B.Cu") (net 6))
 (via (at 157 100) (size 0.6) (drill 0.3) (layers "F.Cu" "B.Cu") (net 6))
 (via (at 151 100) (size 0.6) (drill 0.3) (layers "F.Cu" "B.Cu") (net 6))
 (via (at 156 99) (size 0.6) (drill 0.3) (layers "F.Cu" "B.Cu") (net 6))
 (via (at 153 100) (size 0.6) (drill 0.3) (layers "F.Cu" "B.Cu") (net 6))
 (via (at 158 107) (size 0.6) (drill 0.3) (layers "F.Cu" "B.Cu") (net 6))
 (via (at 154 101) (size 0.6) (drill 0.3) (layers "F.Cu" "B.Cu") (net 6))
 (via (at 151 107) (size 0.6) (drill 0.3) (layers "F.Cu" "B.Cu") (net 6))
 (via (at 152 107) (size 0.6) (drill 0.3) (layers "F.Cu" "B.Cu") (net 6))
 (via (at 155 104) (size 0.6) (drill 0.3) (layers "F.Cu" "B.Cu") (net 6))
 (via (at 150 99) (size 0.6) (drill 0.3) (layers "F.Cu" "B.Cu") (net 6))
 (via (at 152 100) (size 0.6) (drill 0.3) (layers "F.Cu" "B.Cu") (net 6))
 (via (at 150 104) (size 0.6) (drill 0.3) (layers "F.Cu" "B.Cu") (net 6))
 (via (at 155 99) (size 0.6) (drill 0.3) (layers "F.Cu" "B.Cu") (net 6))
 (via (at 150 102) (size 0.6) (drill 0.3) (layers "F.Cu" "B.Cu") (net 6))
 (via (at 152 99) (size 0.6) (drill 0.3) (layers "F.Cu" "B.Cu") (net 6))
 (via (at 158 102) (size 0.6) (drill 0.3) (layers "F.Cu" "B.Cu") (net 6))
 (via (at 159 107) (size 0.6) (drill 0.3) (layers "F.Cu" "B.Cu") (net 6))
 (via (at 155 100) (size 0.6) (drill 0.3) (layers "F.Cu" "B.Cu") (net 6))
 (via (at 153 105) (size 0.6) (drill 0.3) (layers "F.Cu" "B.Cu") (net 6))
 (via (at 150 106) (size 0.6) (drill 0.3) (layers "F.Cu" "B.Cu") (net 6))
 (via (at 152 105) (size 0.6) (drill 0.3) (layers "F.Cu" "B.Cu") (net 6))
 (via (at 158 103) (size 0.6) (drill 0.3) (layers "F.Cu" "B.Cu") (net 6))
 (via (at 159 103) (size 0.6) (drill 0.3) (layers "F.Cu" "B.Cu") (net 6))
 (via (at 155 103) (size 0.6) (drill 0.3) (layers "F.Cu" "B.Cu") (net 6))
 (via (at 153 107) (size 0.6) (drill 0.3) (layers "F.Cu" "B.Cu") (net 6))
 (via (at 150 107) (size 0.6) (drill 0.3) (layers "F.Cu" "B.Cu") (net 6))
 (via (at 153 102) (size 0.6) (drill 0.3) (layers "F.Cu" "B.Cu") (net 6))
 (via (at 159 106) (size 0.6) (drill 0.3) (layers "F.Cu" "B.Cu") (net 6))
 (via (at 157 101) (size 0.6) (drill 0.3) (layers "F.Cu" "B.Cu") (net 6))
 (via (at 149 99) (size 0.6) (drill 0.3) (layers "F.Cu" "B.Cu") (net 6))
 (via (at 157 104) (size 0.6) (drill 0.3) (layers "F.Cu" "B.Cu") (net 6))
 (via (at 150 105) (size 0.6) (drill 0.3) (layers "F.Cu" "B.Cu") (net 6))
 (via (at 150 100) (size 0.6) (drill 0.3) (layers "F.Cu" "B.Cu") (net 6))
 (via (at 157 106) (size 0.6) (drill 0.3) (layers "F.Cu" "B.Cu") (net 6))
 (via (at 152 102) (size 0.6) (drill 0.3) (layers "F.Cu" "B.Cu") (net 6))
 (via (at 159 100) (size 0.6) (drill 0.3) (layers "F.Cu" "B.Cu") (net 6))
 (via (at 149 105) (size 0.6) (drill 0.3) (layers "F.Cu" "B.Cu") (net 6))
 (via (at 157 99) (size 0.6) (drill 0.3) (layers "F.Cu" "B.Cu") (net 6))
 (via (at 153 104) (size 0.6) (drill 0.3) (layers "F.Cu" "B.Cu") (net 6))
 (via (at 155 105) (size 0.6) (drill 0.3) (layers "F.Cu" "B.Cu") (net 6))
 (via (at 156 102) (size 0.6) (drill 0.3) (layers "F.Cu" "B.Cu") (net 6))
 (via (at 149 101) (size 0.6) (drill 0.3) (layers "F.Cu" "B.Cu") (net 6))
 (via (at 158 106) (size 0.6) (drill 0.3) (layers "F.Cu" "B.Cu") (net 6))
 (via (at 149 102) (size 0.6) (drill 0.3) (layers "F.Cu" "B.Cu") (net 6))
 (via (at 149 106) (size 0.6) (drill 0.3) (layers "F.Cu" "B.Cu") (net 6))
 (via (at 154 106) (size 0.6) (drill 0.3) (layers "F.Cu" "B.Cu") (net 6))
 (via (at 155 106) (size 0.6) (drill 0.3) (layers "F.Cu" "B.Cu") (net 6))
 (via (at 151 105) (size 0.6) (drill 0.3) (layers "F.Cu" "B.Cu") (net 6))
 (via (at 156 100) (size 0.6) (drill 0.3) (layers "F.Cu" "B.Cu") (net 6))
 (via (at 149 104) (size 0.6) (drill 0.3) (layers "F.Cu" "B.Cu") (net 6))
 (via (at 156 103) (size 0.6) (drill 0.3) (layers "F.Cu" "B.Cu") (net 6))
 (via (at 153 101) (size 0.6) (drill 0.3) (layers "F.Cu" "B.Cu") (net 6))
 (via (at 150 103) (size 0.6) (drill 0.3) (layers "F.Cu" "B.Cu") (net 6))
 (via (at 152 104) (size 0.6) (drill 0.3) (layers "F.Cu" "B.Cu") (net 6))
 (via (at 149 103) (size 0.6) (drill 0.3) (layers "F.Cu" "B.Cu") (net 6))
 (via (at 157 103) (size 0.6) (drill 0.3) (layers "F.Cu" "B.Cu") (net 6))
 (via (at 153 103) (size 0.6) (drill 0.3) (layers "F.Cu" "B.Cu") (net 6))
 (via (at 158 101) (size 0.6) (drill 0.3) (layers "F.Cu" "B.Cu") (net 6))
 (via (at 156 105) (size 0.6) (drill 0.3) (layers "F.Cu" "B.Cu") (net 6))
 (via (at 152 101) (size 0.6) (drill 0.3) (layers "F.Cu" "B.Cu") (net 6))
 (via (at 154 107) (size 0.6) (drill 0.3) (layers "F.Cu" "B.Cu") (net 6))
 (via (at 159 101) (size 0.6) (drill 0.3) (layers "F.Cu" "B.Cu") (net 6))
 (via (at 157 102) (size 0.6) (drill 0.3) (layers "F.Cu" "B.Cu") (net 6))
 (via (at 158 100) (size 0.6) (drill 0.3) (layers "F.Cu" "B.Cu") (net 6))
 (via (at 151 106) (size 0.6) (drill 0.3) (layers "F.Cu" "B.Cu") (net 6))
 (via (at 151 104) (size 0.6) (drill 0.3) (layers "F.Cu" "B.Cu") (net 6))
 (via (at 156 106) (size 0.6) (drill 0.3) (layers "F.Cu" "B.Cu") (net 6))
 (via (at 158 105) (size 0.6) (drill 0.3) (layers "F.Cu" "B.Cu") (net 6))
 (via (at 151 102) (size 0.6) (drill 0.3) (layers "F.Cu" "B.Cu") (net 6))
 (segment (start 149 105) (end 159 105) (width 1) (layer "B.Cu") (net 6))
 (segment (start 149 103) (end 159 103) (width 1) (layer "B.Cu") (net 6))
 (segment (start 142.5 107) (end 137.5 112) (width 1) (layer "B.Cu") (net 6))
 (segment (start 149 99) (end 159 99) (width 1) (layer "B.Cu") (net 6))
 (segment (start 138 122) (end 144 122) (width 1) (layer "B.Cu") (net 6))
 (segment (start 137.5 112) (end 137.5 121.5) (width 1) (layer "B.Cu") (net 6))
 (segment (start 149 100) (end 159 100) (width 1) (layer "B.Cu") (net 6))
 (segment (start 137.5 121.5) (end 138 122) (width 1) (layer "B.Cu") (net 6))
 (segment (start 149 107) (end 159 107) (width 1) (layer "B.Cu") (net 6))
 (segment (start 149 104) (end 159 104) (width 1) (layer "B.Cu") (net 6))
 (segment (start 149 107) (end 142.5 107) (width 1) (layer "B.Cu") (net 6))
 (segment (start 149 106) (end 159 106) (width 1) (layer "B.Cu") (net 6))
 (segment (start 149 102) (end 159 102) (width 1) (layer "B.Cu") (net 6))
 (segment (start 149 101) (end 159 101) (width 1) (layer "B.Cu") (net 6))
 (segment (start 153.5 126.5) (end 154.5 126.5) (width 1) (layer "F.Cu") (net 7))
 (segment (start 146.5 119.5) (end 153.5 126.5) (width 1) (layer "F.Cu") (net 7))
 (via (at 154.5 126.5) (size 0.6) (drill 0.3) (layers "F.Cu" "B.Cu") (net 7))
 (segment (start 172.775 118.225) (end 164.5 126.5) (width 1) (layer "B.Cu") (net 7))
 (segment (start 173.97 118.225) (end 172.775 118.225) (width 1) (layer "B.Cu") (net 7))
 (segment (start 164.5 126.5) (end 154.5 126.5) (width 1) (layer "B.Cu") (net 7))
 (segment (start 179.05 118.225) (end 179.05 120.233184) (width 1) (layer "F.Cu") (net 4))
 (segment (start 168.6475 122.185) (end 162.4625 116) (width 1) (layer "F.Cu") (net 4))
 (segment (start 177.098184 122.185) (end 168.6475 122.185) (width 1) (layer "F.Cu") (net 4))
 (segment (start 159.0925 112.63) (end 162.4625 116) (width 1) (layer "F.Cu") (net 4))
 (segment (start 179.05 120.233184) (end 177.098184 122.185) (width 1) (layer "F.Cu") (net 4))
 (segment (start 157.4 112.63) (end 159.0925 112.63) (width 1) (layer "F.Cu") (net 4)))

